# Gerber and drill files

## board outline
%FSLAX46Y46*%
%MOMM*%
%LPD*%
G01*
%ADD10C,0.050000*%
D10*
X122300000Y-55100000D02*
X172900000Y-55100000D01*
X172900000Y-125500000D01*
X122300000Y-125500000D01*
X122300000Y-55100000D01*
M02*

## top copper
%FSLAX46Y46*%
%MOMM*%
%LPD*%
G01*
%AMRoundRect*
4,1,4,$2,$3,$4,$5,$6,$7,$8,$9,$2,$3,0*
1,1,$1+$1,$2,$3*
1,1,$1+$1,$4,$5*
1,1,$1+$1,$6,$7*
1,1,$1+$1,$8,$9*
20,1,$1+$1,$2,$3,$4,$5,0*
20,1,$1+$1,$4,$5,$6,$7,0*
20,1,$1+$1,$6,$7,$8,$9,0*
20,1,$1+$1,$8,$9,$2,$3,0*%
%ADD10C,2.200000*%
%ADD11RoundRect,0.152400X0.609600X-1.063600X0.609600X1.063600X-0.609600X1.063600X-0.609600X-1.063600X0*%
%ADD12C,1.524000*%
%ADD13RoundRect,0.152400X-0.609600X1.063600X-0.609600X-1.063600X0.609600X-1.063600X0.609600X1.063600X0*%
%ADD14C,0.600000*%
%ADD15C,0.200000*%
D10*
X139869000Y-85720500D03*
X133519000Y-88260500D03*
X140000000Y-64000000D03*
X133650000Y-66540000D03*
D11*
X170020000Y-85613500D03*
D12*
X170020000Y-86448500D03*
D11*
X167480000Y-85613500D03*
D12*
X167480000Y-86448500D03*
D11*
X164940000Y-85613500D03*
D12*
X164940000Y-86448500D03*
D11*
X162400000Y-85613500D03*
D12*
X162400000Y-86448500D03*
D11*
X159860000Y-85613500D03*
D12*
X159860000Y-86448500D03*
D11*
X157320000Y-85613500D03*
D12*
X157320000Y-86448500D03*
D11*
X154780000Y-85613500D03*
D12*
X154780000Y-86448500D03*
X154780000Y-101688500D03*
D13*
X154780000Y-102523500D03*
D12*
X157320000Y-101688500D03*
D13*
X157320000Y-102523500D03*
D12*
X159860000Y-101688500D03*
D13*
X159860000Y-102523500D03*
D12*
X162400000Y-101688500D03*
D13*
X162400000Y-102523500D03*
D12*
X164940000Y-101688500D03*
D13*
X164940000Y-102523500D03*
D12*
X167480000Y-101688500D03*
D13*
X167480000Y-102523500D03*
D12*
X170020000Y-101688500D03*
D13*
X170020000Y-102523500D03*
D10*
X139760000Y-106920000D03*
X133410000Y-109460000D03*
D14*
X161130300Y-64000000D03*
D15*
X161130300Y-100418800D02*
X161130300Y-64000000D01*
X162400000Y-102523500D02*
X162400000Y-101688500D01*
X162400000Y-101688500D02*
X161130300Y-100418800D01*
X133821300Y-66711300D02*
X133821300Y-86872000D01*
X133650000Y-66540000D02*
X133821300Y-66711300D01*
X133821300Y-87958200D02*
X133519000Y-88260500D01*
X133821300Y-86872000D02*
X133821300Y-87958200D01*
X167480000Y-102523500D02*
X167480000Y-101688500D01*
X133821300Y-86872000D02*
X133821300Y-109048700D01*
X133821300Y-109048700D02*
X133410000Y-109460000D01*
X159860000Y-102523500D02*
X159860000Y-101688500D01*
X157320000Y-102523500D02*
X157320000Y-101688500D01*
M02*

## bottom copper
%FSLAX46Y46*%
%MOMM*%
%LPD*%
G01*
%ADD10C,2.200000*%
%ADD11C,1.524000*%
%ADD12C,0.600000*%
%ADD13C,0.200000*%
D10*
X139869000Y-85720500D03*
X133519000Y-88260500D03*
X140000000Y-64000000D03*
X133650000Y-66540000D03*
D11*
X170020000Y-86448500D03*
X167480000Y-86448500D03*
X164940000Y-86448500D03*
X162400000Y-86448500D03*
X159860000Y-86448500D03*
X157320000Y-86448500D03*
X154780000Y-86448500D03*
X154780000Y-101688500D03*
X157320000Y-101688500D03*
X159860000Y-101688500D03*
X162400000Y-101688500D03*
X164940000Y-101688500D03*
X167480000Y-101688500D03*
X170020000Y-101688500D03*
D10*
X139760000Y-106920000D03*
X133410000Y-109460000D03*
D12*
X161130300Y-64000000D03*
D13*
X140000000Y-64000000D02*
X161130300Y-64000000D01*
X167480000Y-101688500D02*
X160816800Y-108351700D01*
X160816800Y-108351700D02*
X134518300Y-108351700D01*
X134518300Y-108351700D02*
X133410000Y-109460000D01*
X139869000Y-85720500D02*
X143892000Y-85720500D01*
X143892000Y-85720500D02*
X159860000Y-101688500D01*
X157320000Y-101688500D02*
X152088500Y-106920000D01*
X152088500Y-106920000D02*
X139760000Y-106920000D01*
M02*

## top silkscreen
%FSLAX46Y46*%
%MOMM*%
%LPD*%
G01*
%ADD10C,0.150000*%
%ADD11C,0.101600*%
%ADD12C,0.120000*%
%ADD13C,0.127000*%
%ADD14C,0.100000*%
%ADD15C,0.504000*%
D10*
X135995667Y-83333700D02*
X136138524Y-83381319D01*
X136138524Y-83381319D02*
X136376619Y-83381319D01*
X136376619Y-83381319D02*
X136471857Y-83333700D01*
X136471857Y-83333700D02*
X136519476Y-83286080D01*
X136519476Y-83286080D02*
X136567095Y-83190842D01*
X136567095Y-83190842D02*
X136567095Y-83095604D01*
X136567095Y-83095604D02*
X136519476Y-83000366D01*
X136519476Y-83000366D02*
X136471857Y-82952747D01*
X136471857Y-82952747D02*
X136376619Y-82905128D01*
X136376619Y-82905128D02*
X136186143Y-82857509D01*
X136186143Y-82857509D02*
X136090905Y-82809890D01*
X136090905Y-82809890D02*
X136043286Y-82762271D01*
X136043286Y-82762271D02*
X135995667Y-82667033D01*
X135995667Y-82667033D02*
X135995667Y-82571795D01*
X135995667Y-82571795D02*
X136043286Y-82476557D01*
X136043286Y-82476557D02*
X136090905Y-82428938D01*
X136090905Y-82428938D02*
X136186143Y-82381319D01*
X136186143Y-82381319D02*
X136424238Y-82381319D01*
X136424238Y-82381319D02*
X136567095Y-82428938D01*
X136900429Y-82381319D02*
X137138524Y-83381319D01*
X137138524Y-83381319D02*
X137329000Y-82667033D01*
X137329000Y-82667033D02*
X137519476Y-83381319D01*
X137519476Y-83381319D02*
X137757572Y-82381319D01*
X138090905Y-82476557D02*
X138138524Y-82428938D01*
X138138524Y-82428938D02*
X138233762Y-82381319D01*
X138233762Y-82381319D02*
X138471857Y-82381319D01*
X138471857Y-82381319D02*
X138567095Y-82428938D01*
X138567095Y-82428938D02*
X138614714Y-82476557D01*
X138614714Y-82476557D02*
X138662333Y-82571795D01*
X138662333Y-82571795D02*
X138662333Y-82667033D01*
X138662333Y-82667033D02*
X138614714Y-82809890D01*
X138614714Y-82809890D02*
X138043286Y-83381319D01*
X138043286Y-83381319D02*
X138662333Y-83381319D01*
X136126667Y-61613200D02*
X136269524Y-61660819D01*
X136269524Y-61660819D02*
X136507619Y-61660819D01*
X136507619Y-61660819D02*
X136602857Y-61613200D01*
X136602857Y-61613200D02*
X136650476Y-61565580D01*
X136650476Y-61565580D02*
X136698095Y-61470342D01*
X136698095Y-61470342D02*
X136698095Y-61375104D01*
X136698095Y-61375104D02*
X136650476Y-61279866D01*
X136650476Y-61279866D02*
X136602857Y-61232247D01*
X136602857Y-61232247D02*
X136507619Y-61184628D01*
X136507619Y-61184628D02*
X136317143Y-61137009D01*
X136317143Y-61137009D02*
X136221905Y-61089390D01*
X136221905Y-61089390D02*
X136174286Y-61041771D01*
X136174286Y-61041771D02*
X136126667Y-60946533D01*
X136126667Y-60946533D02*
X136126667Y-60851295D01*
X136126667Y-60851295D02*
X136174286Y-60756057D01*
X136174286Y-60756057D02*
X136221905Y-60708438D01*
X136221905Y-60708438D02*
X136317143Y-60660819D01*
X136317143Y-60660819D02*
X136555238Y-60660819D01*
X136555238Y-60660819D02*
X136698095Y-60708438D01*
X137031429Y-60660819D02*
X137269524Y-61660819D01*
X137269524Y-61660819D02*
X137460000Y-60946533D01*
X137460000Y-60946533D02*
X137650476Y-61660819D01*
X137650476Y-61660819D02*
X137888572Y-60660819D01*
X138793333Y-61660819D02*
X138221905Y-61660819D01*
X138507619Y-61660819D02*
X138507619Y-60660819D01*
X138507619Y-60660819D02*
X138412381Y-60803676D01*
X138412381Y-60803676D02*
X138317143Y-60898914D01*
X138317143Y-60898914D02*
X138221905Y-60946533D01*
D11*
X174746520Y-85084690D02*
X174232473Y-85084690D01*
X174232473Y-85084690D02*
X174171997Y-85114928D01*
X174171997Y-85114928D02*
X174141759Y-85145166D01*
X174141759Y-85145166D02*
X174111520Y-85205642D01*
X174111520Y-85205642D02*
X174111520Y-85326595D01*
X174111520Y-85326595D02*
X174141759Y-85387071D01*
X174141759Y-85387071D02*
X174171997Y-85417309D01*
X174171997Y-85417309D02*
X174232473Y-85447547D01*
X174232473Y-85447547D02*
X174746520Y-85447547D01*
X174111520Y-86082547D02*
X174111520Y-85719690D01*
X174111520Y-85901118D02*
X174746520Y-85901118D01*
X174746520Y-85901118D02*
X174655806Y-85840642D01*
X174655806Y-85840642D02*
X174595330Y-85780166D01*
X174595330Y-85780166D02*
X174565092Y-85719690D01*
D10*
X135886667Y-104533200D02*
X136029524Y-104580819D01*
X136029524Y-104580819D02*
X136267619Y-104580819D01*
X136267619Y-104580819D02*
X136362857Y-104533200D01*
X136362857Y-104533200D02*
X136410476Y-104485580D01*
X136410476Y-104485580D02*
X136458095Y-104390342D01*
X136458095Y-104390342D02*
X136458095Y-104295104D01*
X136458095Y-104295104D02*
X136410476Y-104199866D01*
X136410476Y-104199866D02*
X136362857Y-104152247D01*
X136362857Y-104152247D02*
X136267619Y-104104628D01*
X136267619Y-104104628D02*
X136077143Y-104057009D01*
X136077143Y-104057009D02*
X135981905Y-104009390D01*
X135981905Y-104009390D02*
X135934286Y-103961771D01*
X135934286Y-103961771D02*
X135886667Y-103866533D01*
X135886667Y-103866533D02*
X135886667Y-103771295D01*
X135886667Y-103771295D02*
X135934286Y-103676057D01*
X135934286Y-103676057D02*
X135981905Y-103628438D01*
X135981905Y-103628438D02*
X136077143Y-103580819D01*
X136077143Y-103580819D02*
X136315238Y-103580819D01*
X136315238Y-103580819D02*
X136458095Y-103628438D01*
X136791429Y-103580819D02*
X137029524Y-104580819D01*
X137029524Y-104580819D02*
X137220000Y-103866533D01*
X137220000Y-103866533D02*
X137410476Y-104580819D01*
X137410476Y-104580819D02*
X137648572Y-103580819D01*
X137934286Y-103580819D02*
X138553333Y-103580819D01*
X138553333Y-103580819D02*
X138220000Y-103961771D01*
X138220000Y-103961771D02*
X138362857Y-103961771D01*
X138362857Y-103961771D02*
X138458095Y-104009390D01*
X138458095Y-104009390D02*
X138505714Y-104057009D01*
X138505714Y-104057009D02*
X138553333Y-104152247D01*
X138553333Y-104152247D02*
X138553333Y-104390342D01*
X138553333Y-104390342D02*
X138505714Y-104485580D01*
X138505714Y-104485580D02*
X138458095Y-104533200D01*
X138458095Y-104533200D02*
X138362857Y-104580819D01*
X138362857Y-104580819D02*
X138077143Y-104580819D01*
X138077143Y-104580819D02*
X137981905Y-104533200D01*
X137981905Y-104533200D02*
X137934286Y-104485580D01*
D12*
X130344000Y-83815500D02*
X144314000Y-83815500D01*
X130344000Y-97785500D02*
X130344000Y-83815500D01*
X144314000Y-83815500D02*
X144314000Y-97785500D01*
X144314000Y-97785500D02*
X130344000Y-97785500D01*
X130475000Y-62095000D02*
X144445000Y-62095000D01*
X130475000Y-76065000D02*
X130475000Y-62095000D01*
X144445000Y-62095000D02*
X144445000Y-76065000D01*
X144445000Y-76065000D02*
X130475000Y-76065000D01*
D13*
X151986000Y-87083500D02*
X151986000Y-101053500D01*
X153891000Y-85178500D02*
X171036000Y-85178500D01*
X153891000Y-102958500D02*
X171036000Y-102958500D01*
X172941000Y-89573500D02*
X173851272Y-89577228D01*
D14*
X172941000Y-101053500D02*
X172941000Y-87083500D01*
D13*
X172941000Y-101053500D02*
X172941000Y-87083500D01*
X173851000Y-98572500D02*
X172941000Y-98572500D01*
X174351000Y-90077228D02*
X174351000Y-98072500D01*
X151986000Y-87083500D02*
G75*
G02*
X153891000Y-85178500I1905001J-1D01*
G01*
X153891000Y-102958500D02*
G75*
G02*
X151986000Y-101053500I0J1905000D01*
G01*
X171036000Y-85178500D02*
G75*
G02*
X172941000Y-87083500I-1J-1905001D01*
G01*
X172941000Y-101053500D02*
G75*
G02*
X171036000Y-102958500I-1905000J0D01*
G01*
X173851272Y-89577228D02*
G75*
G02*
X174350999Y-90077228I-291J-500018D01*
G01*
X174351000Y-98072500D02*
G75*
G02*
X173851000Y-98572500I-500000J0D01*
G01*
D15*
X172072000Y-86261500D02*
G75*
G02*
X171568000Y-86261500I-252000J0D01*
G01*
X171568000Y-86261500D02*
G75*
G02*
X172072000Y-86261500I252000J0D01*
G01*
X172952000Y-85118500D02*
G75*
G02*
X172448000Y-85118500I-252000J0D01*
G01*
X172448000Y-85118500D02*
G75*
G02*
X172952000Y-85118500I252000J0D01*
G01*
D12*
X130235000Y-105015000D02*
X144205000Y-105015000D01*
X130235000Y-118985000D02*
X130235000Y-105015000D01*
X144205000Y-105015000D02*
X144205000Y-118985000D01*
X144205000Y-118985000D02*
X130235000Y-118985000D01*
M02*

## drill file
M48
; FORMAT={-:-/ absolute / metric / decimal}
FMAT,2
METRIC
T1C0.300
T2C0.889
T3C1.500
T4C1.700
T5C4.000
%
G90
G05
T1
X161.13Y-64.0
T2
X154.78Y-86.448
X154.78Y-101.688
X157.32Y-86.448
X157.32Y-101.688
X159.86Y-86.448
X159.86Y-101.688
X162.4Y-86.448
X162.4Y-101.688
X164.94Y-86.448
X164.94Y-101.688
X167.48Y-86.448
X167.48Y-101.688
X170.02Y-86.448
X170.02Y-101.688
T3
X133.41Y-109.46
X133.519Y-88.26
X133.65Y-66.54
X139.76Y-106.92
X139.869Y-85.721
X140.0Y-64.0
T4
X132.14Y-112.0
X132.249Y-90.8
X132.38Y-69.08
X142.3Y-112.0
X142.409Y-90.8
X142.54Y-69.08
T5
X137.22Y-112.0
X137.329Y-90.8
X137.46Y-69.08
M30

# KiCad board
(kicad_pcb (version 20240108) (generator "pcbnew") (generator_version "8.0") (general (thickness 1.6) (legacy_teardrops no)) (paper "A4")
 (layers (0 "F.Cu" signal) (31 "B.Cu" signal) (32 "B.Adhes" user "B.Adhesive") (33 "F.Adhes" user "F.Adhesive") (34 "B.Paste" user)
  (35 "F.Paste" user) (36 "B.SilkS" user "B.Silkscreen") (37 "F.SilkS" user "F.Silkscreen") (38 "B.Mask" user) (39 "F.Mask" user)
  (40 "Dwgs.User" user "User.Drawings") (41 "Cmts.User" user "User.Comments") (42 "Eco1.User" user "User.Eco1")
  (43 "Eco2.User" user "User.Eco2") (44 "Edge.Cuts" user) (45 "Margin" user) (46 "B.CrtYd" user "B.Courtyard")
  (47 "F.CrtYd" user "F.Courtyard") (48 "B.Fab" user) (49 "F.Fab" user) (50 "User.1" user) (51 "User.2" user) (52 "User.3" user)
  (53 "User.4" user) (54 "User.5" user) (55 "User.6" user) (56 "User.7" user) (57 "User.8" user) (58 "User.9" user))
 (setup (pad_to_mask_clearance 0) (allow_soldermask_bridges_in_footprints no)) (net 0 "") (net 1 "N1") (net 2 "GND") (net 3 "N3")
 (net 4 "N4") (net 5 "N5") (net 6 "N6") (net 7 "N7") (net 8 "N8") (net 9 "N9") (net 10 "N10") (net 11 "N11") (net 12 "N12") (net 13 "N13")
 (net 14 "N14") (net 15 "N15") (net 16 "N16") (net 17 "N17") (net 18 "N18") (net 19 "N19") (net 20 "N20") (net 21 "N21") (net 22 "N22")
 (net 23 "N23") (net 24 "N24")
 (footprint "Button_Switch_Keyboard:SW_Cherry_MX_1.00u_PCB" (layer "F.Cu") (at 139.869 85.7205)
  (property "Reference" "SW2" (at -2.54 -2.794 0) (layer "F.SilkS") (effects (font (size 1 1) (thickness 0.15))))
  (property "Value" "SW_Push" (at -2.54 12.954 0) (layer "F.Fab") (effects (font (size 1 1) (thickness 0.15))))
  (fp_line (start -9.525 -1.905) (end 4.445 -1.905) (stroke (width 0.12) (type solid)) (layer "F.SilkS"))
  (fp_line (start -9.525 12.065) (end -9.525 -1.905) (stroke (width 0.12) (type solid)) (layer "F.SilkS"))
  (fp_line (start 4.445 -1.905) (end 4.445 12.065) (stroke (width 0.12) (type solid)) (layer "F.SilkS"))
  (fp_line (start 4.445 12.065) (end -9.525 12.065) (stroke (width 0.12) (type solid)) (layer "F.SilkS"))
  (pad "" np_thru_hole circle (at -7.62 5.08) (size 1.7 1.7) (drill 1.7) (layers "*.Cu" "*.Mask"))
  (pad "" np_thru_hole circle (at -2.54 5.08) (size 4 4) (drill 4) (layers "*.Cu" "*.Mask"))
  (pad "" np_thru_hole circle (at 2.54 5.08) (size 1.7 1.7) (drill 1.7) (layers "*.Cu" "*.Mask"))
  (pad "1" thru_hole circle (at 0 0) (size 2.2 2.2) (drill 1.5) (layers "*.Cu" "*.Mask") (remove_unused_layers no) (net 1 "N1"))
  (pad "2" thru_hole circle (at -6.35 2.54) (size 2.2 2.2) (drill 1.5) (layers "*.Cu" "*.Mask") (remove_unused_layers no) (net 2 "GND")))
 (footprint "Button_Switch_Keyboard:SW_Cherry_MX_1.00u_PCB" (layer "F.Cu") (at 140 64)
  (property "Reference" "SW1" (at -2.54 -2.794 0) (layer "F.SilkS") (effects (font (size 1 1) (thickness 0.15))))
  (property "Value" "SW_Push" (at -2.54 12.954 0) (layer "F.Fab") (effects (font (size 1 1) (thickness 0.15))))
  (fp_line (start -9.525 -1.905) (end 4.445 -1.905) (stroke (width 0.12) (type solid)) (layer "F.SilkS"))
  (fp_line (start -9.525 12.065) (end -9.525 -1.905) (stroke (width 0.12) (type solid)) (layer "F.SilkS"))
  (fp_line (start 4.445 -1.905) (end 4.445 12.065) (stroke (width 0.12) (type solid)) (layer "F.SilkS"))
  (fp_line (start 4.445 12.065) (end -9.525 12.065) (stroke (width 0.12) (type solid)) (layer "F.SilkS"))
  (pad "" np_thru_hole circle (at -7.62 5.08) (size 1.7 1.7) (drill 1.7) (layers "*.Cu" "*.Mask"))
  (pad "" np_thru_hole circle (at -2.54 5.08) (size 4 4) (drill 4) (layers "*.Cu" "*.Mask"))
  (pad "" np_thru_hole circle (at 2.54 5.08) (size 1.7 1.7) (drill 1.7) (layers "*.Cu" "*.Mask"))
  (pad "1" thru_hole circle (at 0 0) (size 2.2 2.2) (drill 1.5) (layers "*.Cu" "*.Mask") (remove_unused_layers no) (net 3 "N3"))
  (pad "2" thru_hole circle (at -6.35 2.54) (size 2.2 2.2) (drill 1.5) (layers "*.Cu" "*.Mask") (remove_unused_layers no) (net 2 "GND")))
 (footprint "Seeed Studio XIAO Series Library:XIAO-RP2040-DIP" (layer "F.Cu") (at 162.4 94.0685 -90)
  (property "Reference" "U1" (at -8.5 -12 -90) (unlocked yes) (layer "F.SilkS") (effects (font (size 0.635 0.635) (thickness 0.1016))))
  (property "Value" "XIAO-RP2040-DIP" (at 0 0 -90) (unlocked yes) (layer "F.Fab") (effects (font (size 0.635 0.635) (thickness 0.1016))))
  (fp_line (start -6.985 10.414) (end 6.985 10.414) (stroke (width 0.127) (type solid)) (layer "F.SilkS"))
  (fp_line (start -8.89 8.509) (end -8.89 -8.636) (stroke (width 0.127) (type solid)) (layer "F.SilkS"))
  (fp_line (start 8.89 8.509) (end 8.89 -8.636) (stroke (width 0.127) (type solid)) (layer "F.SilkS"))
  (fp_line (start -4.495 -10.541) (end -4.491272 -11.451272) (stroke (width 0.127) (type solid)) (layer "F.SilkS"))
  (fp_line (start 6.985 -10.541) (end -6.985 -10.541) (stroke (width 0.1) (type solid)) (layer "F.SilkS"))
  (fp_line (start 6.985 -10.541) (end -6.985 -10.541) (stroke (width 0.127) (type solid)) (layer "F.SilkS"))
  (fp_line (start 4.504 -11.451) (end 4.504 -10.541) (stroke (width 0.127) (type solid)) (layer "F.SilkS"))
  (fp_line (start -3.991272 -11.951) (end 4.004 -11.951) (stroke (width 0.127) (type solid)) (layer "F.SilkS"))
  (fp_arc (start -6.985 10.414) (mid -8.332038 9.856038) (end -8.89 8.509) (stroke (width 0.127) (type solid)) (layer "F.SilkS"))
  (fp_arc (start 8.89 8.509) (mid 8.332038 9.856038) (end 6.985 10.414) (stroke (width 0.127) (type solid)) (layer "F.SilkS"))
  (fp_arc (start -8.89 -8.636) (mid -8.332038 -9.983038) (end -6.985 -10.541) (stroke (width 0.127) (type solid)) (layer "F.SilkS"))
  (fp_arc (start 6.985 -10.541) (mid 8.332038 -9.983038) (end 8.89 -8.636) (stroke (width 0.127) (type solid)) (layer "F.SilkS"))
  (fp_arc (start -4.491272 -11.451272) (mid -4.344724 -11.804644) (end -3.991272 -11.951) (stroke (width 0.127) (type default))
   (layer "F.SilkS"))
  (fp_arc (start 4.004 -11.951) (mid 4.357553 -11.804553) (end 4.504 -11.451) (stroke (width 0.127) (type default)) (layer "F.SilkS"))
  (fp_circle (center -7.807 -9.42) (end -7.807 -9.674) (stroke (width 0.5) (type solid)) (fill solid) (layer "F.SilkS"))
  (fp_circle (center -8.95 -10.3) (end -8.95 -10.554) (stroke (width 0.5) (type solid)) (fill solid) (layer "F.SilkS"))
  (pad "1" smd roundrect (at -8.455 -7.62 90) (size 2.432 1.524) (layers "F.Cu" "F.Mask") (roundrect_rratio 0.1) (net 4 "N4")
   (thermal_bridge_angle 45))
  (pad "1" thru_hole circle (at -7.62 -7.62 90) (size 1.524 1.524) (drill 0.889) (layers "*.Cu" "*.Mask") (remove_unused_layers no)
   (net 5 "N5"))
  (pad "2" smd roundrect (at -8.455 -5.08 90) (size 2.432 1.524) (layers "F.Cu" "F.Mask") (roundrect_rratio 0.1) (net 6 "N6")
   (thermal_bridge_angle 45))
  (pad "2" thru_hole circle (at -7.62 -5.08 90) (size 1.524 1.524) (drill 0.889) (layers "*.Cu" "*.Mask") (remove_unused_layers no)
   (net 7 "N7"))
  (pad "3" smd roundrect (at -8.455 -2.54 90) (size 2.432 1.524) (layers "F.Cu" "F.Mask") (roundrect_rratio 0.1) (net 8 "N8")
   (thermal_bridge_angle 45))
  (pad "3" thru_hole circle (at -7.62 -2.54 90) (size 1.524 1.524) (drill 0.889) (layers "*.Cu" "*.Mask") (remove_unused_layers no)
   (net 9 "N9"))
  (pad "4" smd roundrect (at -8.455 0 90) (size 2.432 1.524) (layers "F.Cu" "F.Mask") (roundrect_rratio 0.1) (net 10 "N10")
   (thermal_bridge_angle 45))
  (pad "4" thru_hole circle (at -7.62 0 90) (size 1.524 1.524) (drill 0.889) (layers "*.Cu" "*.Mask") (remove_unused_layers no)
   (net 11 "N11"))
  (pad "5" smd roundrect (at -8.455 2.54 90) (size 2.432 1.524) (layers "F.Cu" "F.Mask") (roundrect_rratio 0.1) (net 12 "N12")
   (thermal_bridge_angle 45))
  (pad "5" thru_hole circle (at -7.62 2.54 90) (size 1.524 1.524) (drill 0.889) (layers "*.Cu" "*.Mask") (remove_unused_layers no)
   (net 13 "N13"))
  (pad "6" smd roundrect (at -8.455 5.08 90) (size 2.432 1.524) (layers "F.Cu" "F.Mask") (roundrect_rratio 0.1) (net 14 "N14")
   (thermal_bridge_angle 45))
  (pad "6" thru_hole circle (at -7.62 5.08 90) (size 1.524 1.524) (drill 0.889) (layers "*.Cu" "*.Mask") (remove_unused_layers no)
   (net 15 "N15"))
  (pad "7" smd roundrect (at -8.455 7.62 90) (size 2.432 1.524) (layers "F.Cu" "F.Mask") (roundrect_rratio 0.1) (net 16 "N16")
   (thermal_bridge_angle 45))
  (pad "7" thru_hole circle (at -7.62 7.62 90) (size 1.524 1.524) (drill 0.889) (layers "*.Cu" "*.Mask") (remove_unused_layers no)
   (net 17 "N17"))
  (pad "8" thru_hole circle (at 7.62 7.62 270) (size 1.524 1.524) (drill 0.889) (layers "*.Cu" "*.Mask") (remove_unused_layers no)
   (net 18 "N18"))
  (pad "8" smd roundrect (at 8.455 7.62 270) (size 2.432 1.524) (layers "F.Cu" "F.Mask") (roundrect_rratio 0.1) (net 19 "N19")
   (thermal_bridge_angle 45))
  (pad "9" thru_hole circle (at 7.62 5.08 270) (size 1.524 1.524) (drill 0.889) (layers "*.Cu" "*.Mask") (remove_unused_layers no)
   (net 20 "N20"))
  (pad "9" smd roundrect (at 8.455 5.08 270) (size 2.432 1.524) (layers "F.Cu" "F.Mask") (roundrect_rratio 0.1) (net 20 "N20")
   (thermal_bridge_angle 45))
  (pad "10" thru_hole circle (at 7.62 2.54 270) (size 1.524 1.524) (drill 0.889) (layers "*.Cu" "*.Mask") (remove_unused_layers no)
   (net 1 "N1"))
  (pad "10" smd roundrect (at 8.455 2.54 270) (size 2.432 1.524) (layers "F.Cu" "F.Mask") (roundrect_rratio 0.1) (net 1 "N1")
   (thermal_bridge_angle 45))
  (pad "11" thru_hole circle (at 7.62 0 270) (size 1.524 1.524) (drill 0.889) (layers "*.Cu" "*.Mask") (remove_unused_layers no)
   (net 3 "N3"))
  (pad "11" smd roundrect (at 8.455 0 270) (size 2.432 1.524) (layers "F.Cu" "F.Mask") (roundrect_rratio 0.1) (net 3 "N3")
   (thermal_bridge_angle 45))
  (pad "12" thru_hole circle (at 7.62 -2.54 270) (size 1.524 1.524) (drill 0.889) (layers "*.Cu" "*.Mask") (remove_unused_layers no)
   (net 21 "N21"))
  (pad "12" smd roundrect (at 8.455 -2.54 270) (size 2.432 1.524) (layers "F.Cu" "F.Mask") (roundrect_rratio 0.1) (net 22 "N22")
   (thermal_bridge_angle 45))
  (pad "13" thru_hole circle (at 7.62 -5.08 270) (size 1.524 1.524) (drill 0.889) (layers "*.Cu" "*.Mask") (remove_unused_layers no)
   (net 2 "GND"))
  (pad "13" smd roundrect (at 8.455 -5.08 270) (size 2.432 1.524) (layers "F.Cu" "F.Mask") (roundrect_rratio 0.1) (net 2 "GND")
   (thermal_bridge_angle 45))
  (pad "14" thru_hole circle (at 7.62 -7.62 270) (size 1.524 1.524) (drill 0.889) (layers "*.Cu" "*.Mask") (remove_unused_layers no)
   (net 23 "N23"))
  (pad "14" smd roundrect (at 8.455 -7.62 270) (size 2.432 1.524) (layers "F.Cu" "F.Mask") (roundrect_rratio 0.1) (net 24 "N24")
   (thermal_bridge_angle 45)))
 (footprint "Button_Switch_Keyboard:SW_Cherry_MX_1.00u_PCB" (layer "F.Cu") (at 139.76 106.92)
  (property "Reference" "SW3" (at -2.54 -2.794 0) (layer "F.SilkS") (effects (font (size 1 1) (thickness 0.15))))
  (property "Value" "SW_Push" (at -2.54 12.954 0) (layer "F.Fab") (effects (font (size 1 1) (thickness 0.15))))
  (fp_line (start -9.525 -1.905) (end 4.445 -1.905) (stroke (width 0.12) (type solid)) (layer "F.SilkS"))
  (fp_line (start -9.525 12.065) (end -9.525 -1.905) (stroke (width 0.12) (type solid)) (layer "F.SilkS"))
  (fp_line (start 4.445 -1.905) (end 4.445 12.065) (stroke (width 0.12) (type solid)) (layer "F.SilkS"))
  (fp_line (start 4.445 12.065) (end -9.525 12.065) (stroke (width 0.12) (type solid)) (layer "F.SilkS"))
  (pad "" np_thru_hole circle (at -7.62 5.08) (size 1.7 1.7) (drill 1.7) (layers "*.Cu" "*.Mask"))
  (pad "" np_thru_hole circle (at -2.54 5.08) (size 4 4) (drill 4) (layers "*.Cu" "*.Mask"))
  (pad "" np_thru_hole circle (at 2.54 5.08) (size 1.7 1.7) (drill 1.7) (layers "*.Cu" "*.Mask"))
  (pad "1" thru_hole circle (at 0 0) (size 2.2 2.2) (drill 1.5) (layers "*.Cu" "*.Mask") (remove_unused_layers no) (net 20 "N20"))
  (pad "2" thru_hole circle (at -6.35 2.54) (size 2.2 2.2) (drill 1.5) (layers "*.Cu" "*.Mask") (remove_unused_layers no) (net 2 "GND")))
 (gr_rect (start 122.3 55.1) (end 172.9 125.5) (stroke (width 0.05) (type default)) (fill none) (layer "Edge.Cuts"))
 (segment (start 161.1303 100.4188) (end 161.1303 64) (width 0.2) (layer "F.Cu") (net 3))
 (segment (start 162.4 102.5235) (end 162.4 101.6885) (width 0.2) (layer "F.Cu") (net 3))
 (segment (start 162.4 101.6885) (end 161.1303 100.4188) (width 0.2) (layer "F.Cu") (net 3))
 (via (at 161.1303 64) (size 0.6) (drill 0.3) (layers "F.Cu" "B.Cu") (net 3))
 (segment (start 140 64) (end 161.1303 64) (width 0.2) (layer "B.Cu") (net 3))
 (segment (start 133.8213 66.7113) (end 133.8213 86.872) (width 0.2) (layer "F.Cu") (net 2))
 (segment (start 133.65 66.54) (end 133.8213 66.7113) (width 0.2) (layer "F.Cu") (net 2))
 (segment (start 133.8213 87.9582) (end 133.519 88.2605) (width 0.2) (layer "F.Cu") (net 2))
 (segment (start 133.8213 86.872) (end 133.8213 87.9582) (width 0.2) (layer "F.Cu") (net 2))
 (segment (start 167.48 102.5235) (end 167.48 101.6885) (width 0.2) (layer "F.Cu") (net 2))
 (segment (start 133.8213 86.872) (end 133.8213 109.0487) (width 0.2) (layer "F.Cu") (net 2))
 (segment (start 133.8213 109.0487) (end 133.41 109.46) (width 0.2) (layer "F.Cu") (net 2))
 (segment (start 167.48 101.6885) (end 160.8168 108.3517) (width 0.2) (layer "B.Cu") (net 2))
 (segment (start 160.8168 108.3517) (end 134.5183 108.3517) (width 0.2) (layer "B.Cu") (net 2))
 (segment (start 134.5183 108.3517) (end 133.41 109.46) (width 0.2) (layer "B.Cu") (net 2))
 (segment (start 159.86 102.5235) (end 159.86 101.6885) (width 0.2) (layer "F.Cu") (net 1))
 (segment (start 139.869 85.7205) (end 143.892 85.7205) (width 0.2) (layer "B.Cu") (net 1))
 (segment (start 143.892 85.7205) (end 159.86 101.6885) (width 0.2) (layer "B.Cu") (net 1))
 (segment (start 157.32 102.5235) (end 157.32 101.6885) (width 0.2) (layer "F.Cu") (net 20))
 (segment (start 157.32 101.6885) (end 152.0885 106.92) (width 0.2) (layer "B.Cu") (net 20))
 (segment (start 152.0885 106.92) (end 139.76 106.92) (width 0.2) (layer "B.Cu") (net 20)))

